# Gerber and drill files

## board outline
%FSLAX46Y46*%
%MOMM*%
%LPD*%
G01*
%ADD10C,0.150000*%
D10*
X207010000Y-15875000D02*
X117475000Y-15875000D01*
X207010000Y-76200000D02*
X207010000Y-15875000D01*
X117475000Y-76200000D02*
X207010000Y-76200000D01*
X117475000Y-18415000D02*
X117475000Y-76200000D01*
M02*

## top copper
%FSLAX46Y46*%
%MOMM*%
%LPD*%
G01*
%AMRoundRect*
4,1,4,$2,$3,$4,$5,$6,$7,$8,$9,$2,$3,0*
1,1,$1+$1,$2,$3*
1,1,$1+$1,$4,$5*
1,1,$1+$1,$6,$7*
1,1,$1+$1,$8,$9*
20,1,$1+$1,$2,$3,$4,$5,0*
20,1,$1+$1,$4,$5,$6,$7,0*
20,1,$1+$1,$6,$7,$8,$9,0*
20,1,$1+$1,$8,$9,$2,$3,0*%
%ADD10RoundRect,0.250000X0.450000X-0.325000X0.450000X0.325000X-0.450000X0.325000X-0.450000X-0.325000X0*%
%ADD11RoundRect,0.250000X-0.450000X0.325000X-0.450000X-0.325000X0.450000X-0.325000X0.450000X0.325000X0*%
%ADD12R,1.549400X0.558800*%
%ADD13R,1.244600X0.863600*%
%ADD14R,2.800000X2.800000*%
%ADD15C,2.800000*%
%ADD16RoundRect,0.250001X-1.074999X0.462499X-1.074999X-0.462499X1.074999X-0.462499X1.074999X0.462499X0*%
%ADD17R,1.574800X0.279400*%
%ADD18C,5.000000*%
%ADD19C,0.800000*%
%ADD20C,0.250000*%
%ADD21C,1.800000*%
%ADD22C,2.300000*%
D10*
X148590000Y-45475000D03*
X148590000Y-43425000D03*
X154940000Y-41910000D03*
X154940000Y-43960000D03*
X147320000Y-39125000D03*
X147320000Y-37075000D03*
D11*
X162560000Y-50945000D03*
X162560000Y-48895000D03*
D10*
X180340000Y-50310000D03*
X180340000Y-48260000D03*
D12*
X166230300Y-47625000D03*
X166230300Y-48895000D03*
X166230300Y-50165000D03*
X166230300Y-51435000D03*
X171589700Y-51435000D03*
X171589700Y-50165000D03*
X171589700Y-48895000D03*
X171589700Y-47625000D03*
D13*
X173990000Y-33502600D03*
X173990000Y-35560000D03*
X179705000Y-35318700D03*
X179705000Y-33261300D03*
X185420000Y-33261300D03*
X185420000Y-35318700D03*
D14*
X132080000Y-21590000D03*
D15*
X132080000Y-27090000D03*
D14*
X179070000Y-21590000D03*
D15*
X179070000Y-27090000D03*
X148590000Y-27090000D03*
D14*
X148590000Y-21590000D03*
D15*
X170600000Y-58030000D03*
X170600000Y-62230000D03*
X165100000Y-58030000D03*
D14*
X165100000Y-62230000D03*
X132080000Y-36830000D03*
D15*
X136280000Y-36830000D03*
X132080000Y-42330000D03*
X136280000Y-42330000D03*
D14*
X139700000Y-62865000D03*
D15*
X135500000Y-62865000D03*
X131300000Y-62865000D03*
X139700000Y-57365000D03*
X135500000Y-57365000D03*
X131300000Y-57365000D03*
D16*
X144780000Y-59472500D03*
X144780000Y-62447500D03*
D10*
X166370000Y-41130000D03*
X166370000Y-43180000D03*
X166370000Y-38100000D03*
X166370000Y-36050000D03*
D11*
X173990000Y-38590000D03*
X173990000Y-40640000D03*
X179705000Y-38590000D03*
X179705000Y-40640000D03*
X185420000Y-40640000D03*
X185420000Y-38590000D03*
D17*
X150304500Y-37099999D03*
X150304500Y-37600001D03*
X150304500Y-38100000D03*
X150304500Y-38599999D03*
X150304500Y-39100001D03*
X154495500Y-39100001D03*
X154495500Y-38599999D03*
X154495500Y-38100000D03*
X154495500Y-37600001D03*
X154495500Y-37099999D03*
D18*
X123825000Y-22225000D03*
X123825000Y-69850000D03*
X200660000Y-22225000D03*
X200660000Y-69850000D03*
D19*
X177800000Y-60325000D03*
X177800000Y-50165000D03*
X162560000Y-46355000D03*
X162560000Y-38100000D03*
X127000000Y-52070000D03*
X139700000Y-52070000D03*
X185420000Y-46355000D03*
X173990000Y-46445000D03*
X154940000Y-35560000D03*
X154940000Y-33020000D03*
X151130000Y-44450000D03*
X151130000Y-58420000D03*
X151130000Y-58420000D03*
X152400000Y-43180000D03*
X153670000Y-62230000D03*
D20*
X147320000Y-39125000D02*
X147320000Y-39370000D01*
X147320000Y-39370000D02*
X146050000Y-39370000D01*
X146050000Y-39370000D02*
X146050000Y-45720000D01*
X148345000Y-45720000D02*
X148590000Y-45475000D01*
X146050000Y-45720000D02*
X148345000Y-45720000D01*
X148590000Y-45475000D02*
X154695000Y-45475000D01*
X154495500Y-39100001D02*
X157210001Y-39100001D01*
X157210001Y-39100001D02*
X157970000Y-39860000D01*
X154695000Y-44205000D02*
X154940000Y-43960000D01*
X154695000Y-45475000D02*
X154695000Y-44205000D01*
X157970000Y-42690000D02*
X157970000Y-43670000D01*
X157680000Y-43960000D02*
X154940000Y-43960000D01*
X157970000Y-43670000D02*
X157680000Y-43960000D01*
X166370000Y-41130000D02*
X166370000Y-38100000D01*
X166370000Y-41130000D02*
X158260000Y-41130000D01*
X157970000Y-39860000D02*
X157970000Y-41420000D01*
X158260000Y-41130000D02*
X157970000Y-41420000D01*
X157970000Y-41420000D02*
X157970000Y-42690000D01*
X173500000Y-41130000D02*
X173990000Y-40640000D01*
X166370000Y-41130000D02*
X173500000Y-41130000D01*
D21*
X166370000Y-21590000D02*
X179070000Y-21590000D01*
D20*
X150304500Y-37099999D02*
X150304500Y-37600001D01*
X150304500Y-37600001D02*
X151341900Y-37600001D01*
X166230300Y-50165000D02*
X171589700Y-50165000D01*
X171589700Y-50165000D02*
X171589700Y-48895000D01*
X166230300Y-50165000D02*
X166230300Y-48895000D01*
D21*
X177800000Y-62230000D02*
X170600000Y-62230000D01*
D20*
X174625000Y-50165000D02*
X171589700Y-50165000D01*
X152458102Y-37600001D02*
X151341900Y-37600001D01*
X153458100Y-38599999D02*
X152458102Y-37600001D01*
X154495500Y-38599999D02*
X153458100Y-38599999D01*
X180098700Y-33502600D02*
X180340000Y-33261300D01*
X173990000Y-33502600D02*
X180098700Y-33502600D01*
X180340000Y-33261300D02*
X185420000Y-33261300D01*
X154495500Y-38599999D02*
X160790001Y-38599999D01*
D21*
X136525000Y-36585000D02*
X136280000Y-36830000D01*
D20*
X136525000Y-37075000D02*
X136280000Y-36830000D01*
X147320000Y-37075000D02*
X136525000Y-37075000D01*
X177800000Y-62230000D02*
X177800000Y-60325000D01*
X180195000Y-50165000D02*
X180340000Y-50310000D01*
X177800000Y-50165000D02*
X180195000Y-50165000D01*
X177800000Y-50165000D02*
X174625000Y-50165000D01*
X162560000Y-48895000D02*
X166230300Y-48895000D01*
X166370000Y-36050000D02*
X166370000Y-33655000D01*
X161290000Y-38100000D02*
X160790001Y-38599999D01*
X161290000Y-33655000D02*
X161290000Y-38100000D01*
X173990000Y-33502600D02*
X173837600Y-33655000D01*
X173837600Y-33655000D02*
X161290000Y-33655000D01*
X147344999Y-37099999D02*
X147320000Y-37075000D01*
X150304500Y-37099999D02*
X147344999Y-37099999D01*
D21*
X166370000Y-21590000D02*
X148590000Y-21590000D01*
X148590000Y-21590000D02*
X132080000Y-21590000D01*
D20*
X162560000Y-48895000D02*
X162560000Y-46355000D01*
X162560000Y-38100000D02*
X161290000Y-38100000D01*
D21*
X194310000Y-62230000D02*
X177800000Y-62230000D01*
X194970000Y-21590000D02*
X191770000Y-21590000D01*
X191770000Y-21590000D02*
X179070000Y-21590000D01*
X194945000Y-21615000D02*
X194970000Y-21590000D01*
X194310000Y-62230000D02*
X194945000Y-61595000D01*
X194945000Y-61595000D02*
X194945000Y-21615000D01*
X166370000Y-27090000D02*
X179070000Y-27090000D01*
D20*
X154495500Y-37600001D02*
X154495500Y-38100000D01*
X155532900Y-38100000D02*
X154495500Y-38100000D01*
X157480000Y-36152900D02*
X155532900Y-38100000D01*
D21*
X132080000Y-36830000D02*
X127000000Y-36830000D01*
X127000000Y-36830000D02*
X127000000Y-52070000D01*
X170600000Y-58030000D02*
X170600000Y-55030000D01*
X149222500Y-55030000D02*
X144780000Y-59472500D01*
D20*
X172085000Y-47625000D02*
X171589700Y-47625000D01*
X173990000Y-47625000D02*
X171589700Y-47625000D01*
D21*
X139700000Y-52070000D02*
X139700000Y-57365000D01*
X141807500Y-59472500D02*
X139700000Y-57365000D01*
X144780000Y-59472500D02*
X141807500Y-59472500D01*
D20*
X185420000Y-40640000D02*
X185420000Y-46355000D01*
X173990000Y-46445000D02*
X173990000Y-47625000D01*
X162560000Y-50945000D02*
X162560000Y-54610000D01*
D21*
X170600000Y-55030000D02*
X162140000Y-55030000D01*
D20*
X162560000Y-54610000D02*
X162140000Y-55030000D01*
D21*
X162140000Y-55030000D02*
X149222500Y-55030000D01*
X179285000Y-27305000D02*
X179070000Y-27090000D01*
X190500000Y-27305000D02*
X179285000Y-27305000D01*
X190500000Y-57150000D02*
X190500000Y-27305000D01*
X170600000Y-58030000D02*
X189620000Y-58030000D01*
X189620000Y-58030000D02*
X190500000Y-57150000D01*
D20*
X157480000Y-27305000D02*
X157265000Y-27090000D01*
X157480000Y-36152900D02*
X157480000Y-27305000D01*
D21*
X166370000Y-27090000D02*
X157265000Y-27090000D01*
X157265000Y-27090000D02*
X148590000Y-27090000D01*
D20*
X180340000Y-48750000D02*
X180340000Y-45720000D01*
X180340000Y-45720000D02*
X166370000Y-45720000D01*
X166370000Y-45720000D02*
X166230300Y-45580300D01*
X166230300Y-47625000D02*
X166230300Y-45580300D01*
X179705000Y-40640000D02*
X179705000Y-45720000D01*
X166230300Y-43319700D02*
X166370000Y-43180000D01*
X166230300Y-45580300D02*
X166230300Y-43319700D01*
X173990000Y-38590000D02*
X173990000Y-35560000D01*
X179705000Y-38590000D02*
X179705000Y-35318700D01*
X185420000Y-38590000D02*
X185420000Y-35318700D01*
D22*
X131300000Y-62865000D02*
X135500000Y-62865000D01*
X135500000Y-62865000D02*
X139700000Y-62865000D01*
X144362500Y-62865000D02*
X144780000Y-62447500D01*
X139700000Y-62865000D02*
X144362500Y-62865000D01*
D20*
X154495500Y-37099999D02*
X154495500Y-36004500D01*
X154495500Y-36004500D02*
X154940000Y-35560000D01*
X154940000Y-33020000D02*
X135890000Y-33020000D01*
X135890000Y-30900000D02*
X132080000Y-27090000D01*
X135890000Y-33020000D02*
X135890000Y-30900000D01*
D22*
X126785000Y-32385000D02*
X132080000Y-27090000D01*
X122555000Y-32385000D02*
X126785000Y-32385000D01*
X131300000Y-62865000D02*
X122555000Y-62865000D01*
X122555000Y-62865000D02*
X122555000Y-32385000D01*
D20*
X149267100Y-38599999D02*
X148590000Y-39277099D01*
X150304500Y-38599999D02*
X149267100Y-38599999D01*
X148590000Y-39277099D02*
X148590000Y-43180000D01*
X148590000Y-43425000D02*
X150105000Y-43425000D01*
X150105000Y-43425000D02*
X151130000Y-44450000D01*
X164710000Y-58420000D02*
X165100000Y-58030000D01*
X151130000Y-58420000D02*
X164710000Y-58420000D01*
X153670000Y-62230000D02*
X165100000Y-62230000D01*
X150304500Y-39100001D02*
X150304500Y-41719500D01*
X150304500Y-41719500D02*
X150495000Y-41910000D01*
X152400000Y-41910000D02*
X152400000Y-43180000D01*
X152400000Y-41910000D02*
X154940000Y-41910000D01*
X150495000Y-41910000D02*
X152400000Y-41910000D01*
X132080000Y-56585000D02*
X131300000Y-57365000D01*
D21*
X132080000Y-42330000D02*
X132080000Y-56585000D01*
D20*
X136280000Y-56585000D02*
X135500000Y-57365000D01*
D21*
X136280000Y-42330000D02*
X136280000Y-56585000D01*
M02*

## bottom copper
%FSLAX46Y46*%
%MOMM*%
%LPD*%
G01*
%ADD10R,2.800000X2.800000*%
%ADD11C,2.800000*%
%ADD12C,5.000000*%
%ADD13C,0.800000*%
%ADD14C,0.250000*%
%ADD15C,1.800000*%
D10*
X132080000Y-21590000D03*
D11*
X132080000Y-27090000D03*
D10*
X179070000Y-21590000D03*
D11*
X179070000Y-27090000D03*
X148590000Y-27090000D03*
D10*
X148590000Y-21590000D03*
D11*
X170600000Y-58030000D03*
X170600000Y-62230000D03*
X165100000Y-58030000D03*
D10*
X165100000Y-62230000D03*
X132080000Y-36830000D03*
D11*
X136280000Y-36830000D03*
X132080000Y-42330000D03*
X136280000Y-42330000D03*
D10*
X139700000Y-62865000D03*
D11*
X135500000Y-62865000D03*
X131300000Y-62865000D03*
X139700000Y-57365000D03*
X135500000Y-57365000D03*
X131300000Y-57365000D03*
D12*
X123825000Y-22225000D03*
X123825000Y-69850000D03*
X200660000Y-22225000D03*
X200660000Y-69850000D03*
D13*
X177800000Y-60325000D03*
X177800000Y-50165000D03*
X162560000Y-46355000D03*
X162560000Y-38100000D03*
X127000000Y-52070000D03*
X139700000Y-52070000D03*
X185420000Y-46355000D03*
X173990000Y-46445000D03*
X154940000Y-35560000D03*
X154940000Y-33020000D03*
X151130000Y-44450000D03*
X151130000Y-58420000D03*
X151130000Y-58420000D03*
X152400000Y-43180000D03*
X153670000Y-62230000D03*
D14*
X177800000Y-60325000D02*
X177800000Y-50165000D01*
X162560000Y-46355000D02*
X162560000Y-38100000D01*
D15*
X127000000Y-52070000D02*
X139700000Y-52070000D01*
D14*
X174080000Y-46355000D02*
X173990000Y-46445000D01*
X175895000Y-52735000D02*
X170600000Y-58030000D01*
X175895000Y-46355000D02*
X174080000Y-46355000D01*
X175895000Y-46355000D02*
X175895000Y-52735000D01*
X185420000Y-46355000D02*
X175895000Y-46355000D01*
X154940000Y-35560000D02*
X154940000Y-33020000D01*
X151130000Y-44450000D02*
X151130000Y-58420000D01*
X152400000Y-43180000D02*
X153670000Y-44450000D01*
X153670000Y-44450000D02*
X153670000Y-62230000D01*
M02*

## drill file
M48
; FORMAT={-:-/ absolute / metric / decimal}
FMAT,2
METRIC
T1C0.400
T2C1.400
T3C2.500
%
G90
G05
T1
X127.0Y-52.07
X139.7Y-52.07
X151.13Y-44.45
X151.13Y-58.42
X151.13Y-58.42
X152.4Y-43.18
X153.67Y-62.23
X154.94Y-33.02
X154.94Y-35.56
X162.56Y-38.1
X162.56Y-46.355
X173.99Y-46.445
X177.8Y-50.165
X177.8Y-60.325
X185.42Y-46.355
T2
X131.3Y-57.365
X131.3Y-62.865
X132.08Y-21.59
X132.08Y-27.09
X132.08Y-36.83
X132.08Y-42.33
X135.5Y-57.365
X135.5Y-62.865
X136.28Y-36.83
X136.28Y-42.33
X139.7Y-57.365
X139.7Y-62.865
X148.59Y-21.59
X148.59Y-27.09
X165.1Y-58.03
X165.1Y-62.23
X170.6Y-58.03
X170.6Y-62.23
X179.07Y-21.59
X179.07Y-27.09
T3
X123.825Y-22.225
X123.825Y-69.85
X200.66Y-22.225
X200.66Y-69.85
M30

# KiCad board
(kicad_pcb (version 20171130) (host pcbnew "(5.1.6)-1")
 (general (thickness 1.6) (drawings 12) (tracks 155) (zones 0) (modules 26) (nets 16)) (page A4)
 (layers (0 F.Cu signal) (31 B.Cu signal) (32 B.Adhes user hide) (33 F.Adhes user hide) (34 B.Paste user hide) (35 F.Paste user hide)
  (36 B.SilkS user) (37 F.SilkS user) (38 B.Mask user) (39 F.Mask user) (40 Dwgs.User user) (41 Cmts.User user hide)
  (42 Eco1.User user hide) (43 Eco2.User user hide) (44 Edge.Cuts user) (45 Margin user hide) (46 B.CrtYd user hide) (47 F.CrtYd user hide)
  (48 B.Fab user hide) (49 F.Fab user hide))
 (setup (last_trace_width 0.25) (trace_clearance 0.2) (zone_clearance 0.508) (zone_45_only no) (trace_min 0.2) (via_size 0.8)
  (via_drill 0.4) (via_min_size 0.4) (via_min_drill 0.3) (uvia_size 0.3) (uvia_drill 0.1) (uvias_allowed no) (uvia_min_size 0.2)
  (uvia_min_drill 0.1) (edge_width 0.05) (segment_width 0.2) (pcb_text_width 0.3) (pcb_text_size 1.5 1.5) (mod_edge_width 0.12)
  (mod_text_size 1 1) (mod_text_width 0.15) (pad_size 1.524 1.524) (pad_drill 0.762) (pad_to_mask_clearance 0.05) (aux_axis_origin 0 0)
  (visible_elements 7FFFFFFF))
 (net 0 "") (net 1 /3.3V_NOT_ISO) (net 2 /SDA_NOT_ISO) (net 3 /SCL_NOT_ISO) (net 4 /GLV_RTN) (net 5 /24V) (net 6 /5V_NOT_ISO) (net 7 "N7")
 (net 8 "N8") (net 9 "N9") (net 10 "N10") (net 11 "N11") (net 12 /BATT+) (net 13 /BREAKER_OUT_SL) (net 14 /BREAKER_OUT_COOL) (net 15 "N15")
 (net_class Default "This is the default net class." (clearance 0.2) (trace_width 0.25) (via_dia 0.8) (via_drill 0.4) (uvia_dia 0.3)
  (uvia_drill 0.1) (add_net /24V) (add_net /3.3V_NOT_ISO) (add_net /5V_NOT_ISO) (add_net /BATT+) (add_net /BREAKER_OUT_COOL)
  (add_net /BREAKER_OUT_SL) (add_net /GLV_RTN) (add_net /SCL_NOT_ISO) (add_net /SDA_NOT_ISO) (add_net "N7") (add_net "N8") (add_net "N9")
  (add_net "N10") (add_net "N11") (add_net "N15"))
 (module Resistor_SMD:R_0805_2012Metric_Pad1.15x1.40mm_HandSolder (layer F.Cu) (at 148.59 44.45 90)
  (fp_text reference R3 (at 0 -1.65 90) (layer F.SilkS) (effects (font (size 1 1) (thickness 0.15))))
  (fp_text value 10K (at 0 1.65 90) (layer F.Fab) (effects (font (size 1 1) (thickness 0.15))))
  (pad 1 smd roundrect (at -1.025 0 90) (size 1.15 1.4) (layers F.Cu F.Paste F.Mask) (roundrect_rratio 0.217391) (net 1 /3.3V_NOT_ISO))
  (pad 2 smd roundrect (at 1.025 0 90) (size 1.15 1.4) (layers F.Cu F.Paste F.Mask) (roundrect_rratio 0.217391) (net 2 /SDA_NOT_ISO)))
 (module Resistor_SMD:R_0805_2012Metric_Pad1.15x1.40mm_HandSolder (layer F.Cu) (at 154.94 42.935 90)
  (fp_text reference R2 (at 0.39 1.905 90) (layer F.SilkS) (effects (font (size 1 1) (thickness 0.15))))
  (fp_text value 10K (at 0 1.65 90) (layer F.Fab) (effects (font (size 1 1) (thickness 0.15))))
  (pad 2 smd roundrect (at 1.025 0 90) (size 1.15 1.4) (layers F.Cu F.Paste F.Mask) (roundrect_rratio 0.217391) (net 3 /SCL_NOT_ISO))
  (pad 1 smd roundrect (at -1.025 0 90) (size 1.15 1.4) (layers F.Cu F.Paste F.Mask) (roundrect_rratio 0.217391) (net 1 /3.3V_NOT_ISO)))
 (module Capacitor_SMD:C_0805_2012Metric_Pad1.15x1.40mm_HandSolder (layer F.Cu) (at 147.32 38.1 90)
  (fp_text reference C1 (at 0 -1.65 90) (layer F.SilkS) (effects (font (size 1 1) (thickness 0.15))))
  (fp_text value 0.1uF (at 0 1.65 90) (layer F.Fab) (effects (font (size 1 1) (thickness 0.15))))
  (pad 1 smd roundrect (at -1.025 0 90) (size 1.15 1.4) (layers F.Cu F.Paste F.Mask) (roundrect_rratio 0.217391) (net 1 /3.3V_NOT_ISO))
  (pad 2 smd roundrect (at 1.025 0 90) (size 1.15 1.4) (layers F.Cu F.Paste F.Mask) (roundrect_rratio 0.217391) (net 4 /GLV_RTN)))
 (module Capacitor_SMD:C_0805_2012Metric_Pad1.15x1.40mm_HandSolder (layer F.Cu) (at 162.56 49.92 270)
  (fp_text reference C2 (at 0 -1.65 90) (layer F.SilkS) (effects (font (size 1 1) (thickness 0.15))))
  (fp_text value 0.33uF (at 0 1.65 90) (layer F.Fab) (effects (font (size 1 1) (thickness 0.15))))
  (pad 2 smd roundrect (at 1.025 0 270) (size 1.15 1.4) (layers F.Cu F.Paste F.Mask) (roundrect_rratio 0.217391) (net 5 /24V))
  (pad 1 smd roundrect (at -1.025 0 270) (size 1.15 1.4) (layers F.Cu F.Paste F.Mask) (roundrect_rratio 0.217391) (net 4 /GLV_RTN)))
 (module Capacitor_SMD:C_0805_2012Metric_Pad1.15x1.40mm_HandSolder (layer F.Cu) (at 180.34 49.285 90)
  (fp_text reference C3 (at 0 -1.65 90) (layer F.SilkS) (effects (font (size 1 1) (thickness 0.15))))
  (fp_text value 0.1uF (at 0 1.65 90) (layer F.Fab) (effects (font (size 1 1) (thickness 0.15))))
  (pad 1 smd roundrect (at -1.025 0 90) (size 1.15 1.4) (layers F.Cu F.Paste F.Mask) (roundrect_rratio 0.217391) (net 4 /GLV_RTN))
  (pad 2 smd roundrect (at 1.025 0 90) (size 1.15 1.4) (layers F.Cu F.Paste F.Mask) (roundrect_rratio 0.217391) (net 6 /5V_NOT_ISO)))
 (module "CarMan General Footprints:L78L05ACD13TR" (layer F.Cu) (at 168.91 49.53)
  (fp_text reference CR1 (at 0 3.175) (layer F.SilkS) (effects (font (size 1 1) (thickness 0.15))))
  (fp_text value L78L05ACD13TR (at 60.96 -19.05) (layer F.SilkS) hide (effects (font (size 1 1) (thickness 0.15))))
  (pad 1 smd rect (at -2.6797 -1.905) (size 1.5494 0.5588) (layers F.Cu F.Paste F.Mask) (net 6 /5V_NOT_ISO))
  (pad 2 smd rect (at -2.6797 -0.635) (size 1.5494 0.5588) (layers F.Cu F.Paste F.Mask) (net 4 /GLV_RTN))
  (pad 3 smd rect (at -2.6797 0.635) (size 1.5494 0.5588) (layers F.Cu F.Paste F.Mask) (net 4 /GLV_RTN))
  (pad 4 smd rect (at -2.6797 1.905) (size 1.5494 0.5588) (layers F.Cu F.Paste F.Mask) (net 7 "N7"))
  (pad 5 smd rect (at 2.6797 1.905) (size 1.5494 0.5588) (layers F.Cu F.Paste F.Mask) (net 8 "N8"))
  (pad 6 smd rect (at 2.6797 0.635) (size 1.5494 0.5588) (layers F.Cu F.Paste F.Mask) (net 4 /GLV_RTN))
  (pad 7 smd rect (at 2.6797 -0.635) (size 1.5494 0.5588) (layers F.Cu F.Paste F.Mask) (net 4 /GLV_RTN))
  (pad 8 smd rect (at 2.6797 -1.905) (size 1.5494 0.5588) (layers F.Cu F.Paste F.Mask) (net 5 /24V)))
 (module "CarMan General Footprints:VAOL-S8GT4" (layer F.Cu) (at 173.99 34.5313 270)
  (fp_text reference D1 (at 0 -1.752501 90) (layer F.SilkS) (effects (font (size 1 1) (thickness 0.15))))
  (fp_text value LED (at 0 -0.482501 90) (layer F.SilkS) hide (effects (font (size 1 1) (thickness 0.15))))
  (pad 1 smd rect (at -1.0287 0 270) (size 0.8636 1.2446) (layers F.Cu F.Paste F.Mask) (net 4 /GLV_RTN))
  (pad 2 smd rect (at 1.0287 0 270) (size 0.8636 1.2446) (layers F.Cu F.Paste F.Mask) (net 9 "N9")))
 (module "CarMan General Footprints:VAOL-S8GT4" (layer F.Cu) (at 179.705 34.29 270)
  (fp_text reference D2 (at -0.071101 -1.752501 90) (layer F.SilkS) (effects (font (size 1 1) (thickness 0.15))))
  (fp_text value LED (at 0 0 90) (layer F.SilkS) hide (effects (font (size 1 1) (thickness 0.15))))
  (pad 2 smd rect (at 1.0287 0 270) (size 0.8636 1.2446) (layers F.Cu F.Paste F.Mask) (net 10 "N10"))
  (pad 1 smd rect (at -1.0287 0 270) (size 0.8636 1.2446) (layers F.Cu F.Paste F.Mask) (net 4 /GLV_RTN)))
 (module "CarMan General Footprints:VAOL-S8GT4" (layer F.Cu) (at 185.42 34.29 270)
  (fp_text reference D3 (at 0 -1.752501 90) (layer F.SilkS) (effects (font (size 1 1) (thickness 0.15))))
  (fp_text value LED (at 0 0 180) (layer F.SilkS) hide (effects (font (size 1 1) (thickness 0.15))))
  (pad 1 smd rect (at -1.0287 0 270) (size 0.8636 1.2446) (layers F.Cu F.Paste F.Mask) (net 4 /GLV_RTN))
  (pad 2 smd rect (at 1.0287 0 270) (size 0.8636 1.2446) (layers F.Cu F.Paste F.Mask) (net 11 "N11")))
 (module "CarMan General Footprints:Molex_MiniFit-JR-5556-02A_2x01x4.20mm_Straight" (layer F.Cu) (at 132.08 21.59)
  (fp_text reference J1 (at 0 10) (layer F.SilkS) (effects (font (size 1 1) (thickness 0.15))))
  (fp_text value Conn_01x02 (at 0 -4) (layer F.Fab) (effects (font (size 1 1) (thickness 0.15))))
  (pad 1 thru_hole rect (at 0 0) (size 2.8 2.8) (drill 1.4) (layers *.Cu *.Mask) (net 4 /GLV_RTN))
  (pad 2 thru_hole circle (at 0 5.5) (size 2.8 2.8) (drill 1.4) (layers *.Cu *.Mask) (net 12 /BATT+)))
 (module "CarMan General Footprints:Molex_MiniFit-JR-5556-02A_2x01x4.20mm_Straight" (layer F.Cu) (at 179.07 21.59)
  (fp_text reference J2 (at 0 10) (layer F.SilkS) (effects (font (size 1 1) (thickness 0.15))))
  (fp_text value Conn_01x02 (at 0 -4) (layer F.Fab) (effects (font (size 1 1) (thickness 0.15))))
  (pad 1 thru_hole rect (at 0 0) (size 2.8 2.8) (drill 1.4) (layers *.Cu *.Mask) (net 4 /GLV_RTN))
  (pad 2 thru_hole circle (at 0 5.5) (size 2.8 2.8) (drill 1.4) (layers *.Cu *.Mask) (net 5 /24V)))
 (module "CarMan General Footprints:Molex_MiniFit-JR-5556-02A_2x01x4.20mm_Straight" (layer F.Cu) (at 148.59 21.59)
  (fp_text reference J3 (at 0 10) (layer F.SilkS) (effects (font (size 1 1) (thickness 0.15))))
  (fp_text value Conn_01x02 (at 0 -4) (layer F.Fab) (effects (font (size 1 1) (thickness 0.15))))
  (pad 2 thru_hole circle (at 0 5.5) (size 2.8 2.8) (drill 1.4) (layers *.Cu *.Mask) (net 5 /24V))
  (pad 1 thru_hole rect (at 0 0) (size 2.8 2.8) (drill 1.4) (layers *.Cu *.Mask) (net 4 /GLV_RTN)))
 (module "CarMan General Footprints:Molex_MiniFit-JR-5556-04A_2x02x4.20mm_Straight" (layer F.Cu) (at 165.1 62.23 90)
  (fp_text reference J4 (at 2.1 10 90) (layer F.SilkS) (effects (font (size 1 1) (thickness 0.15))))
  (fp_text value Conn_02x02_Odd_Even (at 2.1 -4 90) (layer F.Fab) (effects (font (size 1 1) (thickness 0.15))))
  (pad 4 thru_hole circle (at 4.2 5.5 90) (size 2.8 2.8) (drill 1.4) (layers *.Cu *.Mask) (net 5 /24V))
  (pad 3 thru_hole circle (at 0 5.5 90) (size 2.8 2.8) (drill 1.4) (layers *.Cu *.Mask) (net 4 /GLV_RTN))
  (pad 2 thru_hole circle (at 4.2 0 90) (size 2.8 2.8) (drill 1.4) (layers *.Cu *.Mask) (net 2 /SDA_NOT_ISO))
  (pad 1 thru_hole rect (at 0 0 90) (size 2.8 2.8) (drill 1.4) (layers *.Cu *.Mask) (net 3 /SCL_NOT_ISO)))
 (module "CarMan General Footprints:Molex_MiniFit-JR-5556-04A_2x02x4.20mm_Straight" (layer F.Cu) (at 132.08 36.83)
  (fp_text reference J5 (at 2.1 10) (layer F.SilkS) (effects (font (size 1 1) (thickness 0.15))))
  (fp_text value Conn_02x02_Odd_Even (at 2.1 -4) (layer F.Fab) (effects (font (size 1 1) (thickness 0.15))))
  (pad 1 thru_hole rect (at 0 0) (size 2.8 2.8) (drill 1.4) (layers *.Cu *.Mask) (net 5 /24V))
  (pad 2 thru_hole circle (at 4.2 0) (size 2.8 2.8) (drill 1.4) (layers *.Cu *.Mask) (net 4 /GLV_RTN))
  (pad 3 thru_hole circle (at 0 5.5) (size 2.8 2.8) (drill 1.4) (layers *.Cu *.Mask) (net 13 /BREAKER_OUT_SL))
  (pad 4 thru_hole circle (at 4.2 5.5) (size 2.8 2.8) (drill 1.4) (layers *.Cu *.Mask) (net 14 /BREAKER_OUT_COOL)))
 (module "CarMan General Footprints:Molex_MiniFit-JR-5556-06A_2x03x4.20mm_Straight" (layer F.Cu) (at 139.7 62.865 180)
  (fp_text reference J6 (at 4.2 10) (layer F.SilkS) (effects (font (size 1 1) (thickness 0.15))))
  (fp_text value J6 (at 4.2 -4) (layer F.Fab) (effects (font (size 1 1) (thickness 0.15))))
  (pad 1 thru_hole rect (at 0 0 180) (size 2.8 2.8) (drill 1.4) (layers *.Cu *.Mask) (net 12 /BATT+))
  (pad 2 thru_hole circle (at 4.2 0 180) (size 2.8 2.8) (drill 1.4) (layers *.Cu *.Mask) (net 12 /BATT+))
  (pad 3 thru_hole circle (at 8.4 0 180) (size 2.8 2.8) (drill 1.4) (layers *.Cu *.Mask) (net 12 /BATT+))
  (pad 4 thru_hole circle (at 0 5.5 180) (size 2.8 2.8) (drill 1.4) (layers *.Cu *.Mask) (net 5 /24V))
  (pad 5 thru_hole circle (at 4.2 5.5 180) (size 2.8 2.8) (drill 1.4) (layers *.Cu *.Mask) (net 14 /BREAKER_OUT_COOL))
  (pad 6 thru_hole circle (at 8.4 5.5 180) (size 2.8 2.8) (drill 1.4) (layers *.Cu *.Mask) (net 13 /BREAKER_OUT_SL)))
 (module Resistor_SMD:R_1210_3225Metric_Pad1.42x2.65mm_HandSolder (layer F.Cu) (at 144.78 60.96 270)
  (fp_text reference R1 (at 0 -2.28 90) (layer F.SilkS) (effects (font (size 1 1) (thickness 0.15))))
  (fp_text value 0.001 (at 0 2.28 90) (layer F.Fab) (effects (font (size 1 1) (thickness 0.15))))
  (pad 1 smd roundrect (at -1.4875 0 270) (size 1.425 2.65) (layers F.Cu F.Paste F.Mask) (roundrect_rratio 0.175439) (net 5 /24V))
  (pad 2 smd roundrect (at 1.4875 0 270) (size 1.425 2.65) (layers F.Cu F.Paste F.Mask) (roundrect_rratio 0.175439) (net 12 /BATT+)))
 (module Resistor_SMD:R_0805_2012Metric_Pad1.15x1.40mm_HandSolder (layer F.Cu) (at 166.37 42.155 90)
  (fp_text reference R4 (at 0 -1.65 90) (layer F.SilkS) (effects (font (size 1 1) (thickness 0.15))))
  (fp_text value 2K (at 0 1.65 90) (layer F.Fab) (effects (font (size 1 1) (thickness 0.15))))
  (pad 2 smd roundrect (at 1.025 0 90) (size 1.15 1.4) (layers F.Cu F.Paste F.Mask) (roundrect_rratio 0.217391) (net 1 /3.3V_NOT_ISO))
  (pad 1 smd roundrect (at -1.025 0 90) (size 1.15 1.4) (layers F.Cu F.Paste F.Mask) (roundrect_rratio 0.217391) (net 6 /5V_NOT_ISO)))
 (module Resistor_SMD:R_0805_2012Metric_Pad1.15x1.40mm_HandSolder (layer F.Cu) (at 166.37 37.075 90)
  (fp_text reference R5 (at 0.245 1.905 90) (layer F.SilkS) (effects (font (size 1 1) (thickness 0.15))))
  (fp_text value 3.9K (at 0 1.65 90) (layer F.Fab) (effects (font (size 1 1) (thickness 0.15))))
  (pad 1 smd roundrect (at -1.025 0 90) (size 1.15 1.4) (layers F.Cu F.Paste F.Mask) (roundrect_rratio 0.217391) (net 1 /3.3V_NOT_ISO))
  (pad 2 smd roundrect (at 1.025 0 90) (size 1.15 1.4) (layers F.Cu F.Paste F.Mask) (roundrect_rratio 0.217391) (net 4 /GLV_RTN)))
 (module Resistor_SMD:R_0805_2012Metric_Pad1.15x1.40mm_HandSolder (layer F.Cu) (at 173.99 39.615 270)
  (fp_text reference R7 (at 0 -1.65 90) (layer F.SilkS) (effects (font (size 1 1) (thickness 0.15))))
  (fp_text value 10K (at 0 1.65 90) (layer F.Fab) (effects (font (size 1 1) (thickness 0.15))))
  (pad 1 smd roundrect (at -1.025 0 270) (size 1.15 1.4) (layers F.Cu F.Paste F.Mask) (roundrect_rratio 0.217391) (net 9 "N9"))
  (pad 2 smd roundrect (at 1.025 0 270) (size 1.15 1.4) (layers F.Cu F.Paste F.Mask) (roundrect_rratio 0.217391) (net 1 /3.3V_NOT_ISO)))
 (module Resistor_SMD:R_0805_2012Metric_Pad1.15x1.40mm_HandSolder (layer F.Cu) (at 179.705 39.615 270)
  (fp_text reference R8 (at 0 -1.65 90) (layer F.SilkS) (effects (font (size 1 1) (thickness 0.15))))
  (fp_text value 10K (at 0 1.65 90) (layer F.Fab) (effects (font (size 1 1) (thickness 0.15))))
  (pad 1 smd roundrect (at -1.025 0 270) (size 1.15 1.4) (layers F.Cu F.Paste F.Mask) (roundrect_rratio 0.217391) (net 10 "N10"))
  (pad 2 smd roundrect (at 1.025 0 270) (size 1.15 1.4) (layers F.Cu F.Paste F.Mask) (roundrect_rratio 0.217391) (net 6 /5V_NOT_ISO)))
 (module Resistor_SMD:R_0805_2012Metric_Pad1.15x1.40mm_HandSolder (layer F.Cu) (at 185.42 39.615 270)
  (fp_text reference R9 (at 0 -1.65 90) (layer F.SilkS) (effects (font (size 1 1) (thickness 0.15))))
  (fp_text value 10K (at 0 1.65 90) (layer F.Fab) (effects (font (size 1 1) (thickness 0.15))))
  (pad 2 smd roundrect (at 1.025 0 270) (size 1.15 1.4) (layers F.Cu F.Paste F.Mask) (roundrect_rratio 0.217391) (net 5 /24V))
  (pad 1 smd roundrect (at -1.025 0 270) (size 1.15 1.4) (layers F.Cu F.Paste F.Mask) (roundrect_rratio 0.217391) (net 11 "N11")))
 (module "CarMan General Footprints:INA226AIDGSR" (layer F.Cu) (at 152.4 38.1)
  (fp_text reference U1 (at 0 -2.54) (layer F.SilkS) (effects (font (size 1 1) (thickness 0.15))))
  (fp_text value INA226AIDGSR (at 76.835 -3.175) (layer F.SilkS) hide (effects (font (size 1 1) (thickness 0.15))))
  (pad 1 smd rect (at -2.0955 -1.000001) (size 1.5748 0.2794) (layers F.Cu F.Paste F.Mask) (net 4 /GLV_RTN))
  (pad 2 smd rect (at -2.0955 -0.499999) (size 1.5748 0.2794) (layers F.Cu F.Paste F.Mask) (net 4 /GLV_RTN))
  (pad 3 smd rect (at -2.0955 0) (size 1.5748 0.2794) (layers F.Cu F.Paste F.Mask) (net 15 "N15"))
  (pad 4 smd rect (at -2.0955 0.499999) (size 1.5748 0.2794) (layers F.Cu F.Paste F.Mask) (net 2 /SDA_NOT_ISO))
  (pad 5 smd rect (at -2.0955 1.000001) (size 1.5748 0.2794) (layers F.Cu F.Paste F.Mask) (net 3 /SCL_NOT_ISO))
  (pad 6 smd rect (at 2.0955 1.000001) (size 1.5748 0.2794) (layers F.Cu F.Paste F.Mask) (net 1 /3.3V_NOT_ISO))
  (pad 7 smd rect (at 2.0955 0.499999) (size 1.5748 0.2794) (layers F.Cu F.Paste F.Mask) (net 4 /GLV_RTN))
  (pad 8 smd rect (at 2.0955 0) (size 1.5748 0.2794) (layers F.Cu F.Paste F.Mask) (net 5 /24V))
  (pad 9 smd rect (at 2.0955 -0.499999) (size 1.5748 0.2794) (layers F.Cu F.Paste F.Mask) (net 5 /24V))
  (pad 10 smd rect (at 2.0955 -1.000001) (size 1.5748 0.2794) (layers F.Cu F.Paste F.Mask) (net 12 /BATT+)))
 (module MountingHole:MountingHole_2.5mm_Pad (layer F.Cu) (at 123.825 22.225)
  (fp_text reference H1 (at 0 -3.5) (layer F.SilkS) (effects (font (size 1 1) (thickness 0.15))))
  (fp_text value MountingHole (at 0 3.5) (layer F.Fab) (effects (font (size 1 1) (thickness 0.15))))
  (pad 1 thru_hole circle (at 0 0) (size 5 5) (drill 2.5) (layers *.Cu *.Mask)))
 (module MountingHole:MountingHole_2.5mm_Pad (layer F.Cu) (at 123.825 69.85)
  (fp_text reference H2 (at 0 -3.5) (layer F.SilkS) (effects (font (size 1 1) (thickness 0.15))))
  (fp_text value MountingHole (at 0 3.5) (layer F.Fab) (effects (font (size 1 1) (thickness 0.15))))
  (pad 1 thru_hole circle (at 0 0) (size 5 5) (drill 2.5) (layers *.Cu *.Mask)))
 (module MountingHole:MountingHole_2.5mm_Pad (layer F.Cu) (at 200.66 22.225)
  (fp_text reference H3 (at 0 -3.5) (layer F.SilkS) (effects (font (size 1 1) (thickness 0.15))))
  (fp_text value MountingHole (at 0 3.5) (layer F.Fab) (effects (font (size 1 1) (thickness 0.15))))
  (pad 1 thru_hole circle (at 0 0) (size 5 5) (drill 2.5) (layers *.Cu *.Mask)))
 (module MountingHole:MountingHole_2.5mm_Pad (layer F.Cu) (at 200.66 69.85)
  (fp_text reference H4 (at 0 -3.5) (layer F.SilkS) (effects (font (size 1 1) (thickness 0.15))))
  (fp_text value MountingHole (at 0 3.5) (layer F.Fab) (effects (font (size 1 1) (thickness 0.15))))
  (pad 1 thru_hole circle (at 0 0) (size 5 5) (drill 2.5) (layers *.Cu *.Mask)))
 (gr_line (start 207.01 15.875) (end 117.475 15.875) (layer Edge.Cuts) (width 0.15))
 (gr_line (start 207.01 76.2) (end 207.01 15.875) (layer Edge.Cuts) (width 0.15))
 (gr_line (start 117.475 76.2) (end 207.01 76.2) (layer Edge.Cuts) (width 0.15))
 (gr_line (start 117.475 18.415) (end 117.475 76.2) (layer Edge.Cuts) (width 0.15))
 (segment (start 147.32 39.125) (end 147.32 39.37) (width 0.25) (layer F.Cu) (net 1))
 (segment (start 147.32 39.37) (end 146.05 39.37) (width 0.25) (layer F.Cu) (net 1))
 (segment (start 146.05 39.37) (end 146.05 45.72) (width 0.25) (layer F.Cu) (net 1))
 (segment (start 148.345 45.72) (end 148.59 45.475) (width 0.25) (layer F.Cu) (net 1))
 (segment (start 146.05 45.72) (end 148.345 45.72) (width 0.25) (layer F.Cu) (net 1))
 (segment (start 148.59 45.475) (end 154.695 45.475) (width 0.25) (layer F.Cu) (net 1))
 (segment (start 154.4955 39.100001) (end 157.210001 39.100001) (width 0.25) (layer F.Cu) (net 1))
 (segment (start 157.210001 39.100001) (end 157.97 39.86) (width 0.25) (layer F.Cu) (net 1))
 (segment (start 154.695 44.205) (end 154.94 43.96) (width 0.25) (layer F.Cu) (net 1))
 (segment (start 154.695 45.475) (end 154.695 44.205) (width 0.25) (layer F.Cu) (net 1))
 (segment (start 157.97 42.69) (end 157.97 43.67) (width 0.25) (layer F.Cu) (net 1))
 (segment (start 157.68 43.96) (end 154.94 43.96) (width 0.25) (layer F.Cu) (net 1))
 (segment (start 157.97 43.67) (end 157.68 43.96) (width 0.25) (layer F.Cu) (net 1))
 (segment (start 166.37 41.13) (end 166.37 38.1) (width 0.25) (layer F.Cu) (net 1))
 (segment (start 166.37 41.13) (end 158.26 41.13) (width 0.25) (layer F.Cu) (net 1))
 (segment (start 157.97 39.86) (end 157.97 41.42) (width 0.25) (layer F.Cu) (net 1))
 (segment (start 158.26 41.13) (end 157.97 41.42) (width 0.25) (layer F.Cu) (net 1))
 (segment (start 157.97 41.42) (end 157.97 42.69) (width 0.25) (layer F.Cu) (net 1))
 (segment (start 173.5 41.13) (end 173.99 40.64) (width 0.25) (layer F.Cu) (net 1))
 (segment (start 166.37 41.13) (end 173.5 41.13) (width 0.25) (layer F.Cu) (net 1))
 (segment (start 166.37 21.59) (end 179.07 21.59) (width 1.8) (layer F.Cu) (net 4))
 (segment (start 150.3045 37.099999) (end 150.3045 37.600001) (width 0.25) (layer F.Cu) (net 4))
 (segment (start 150.3045 37.600001) (end 151.3419 37.600001) (width 0.25) (layer F.Cu) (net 4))
 (segment (start 166.2303 50.165) (end 171.5897 50.165) (width 0.25) (layer F.Cu) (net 4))
 (segment (start 171.5897 50.165) (end 171.5897 48.895) (width 0.25) (layer F.Cu) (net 4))
 (segment (start 166.2303 50.165) (end 166.2303 48.895) (width 0.25) (layer F.Cu) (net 4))
 (segment (start 177.8 62.23) (end 170.6 62.23) (width 1.8) (layer F.Cu) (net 4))
 (segment (start 174.625 50.165) (end 171.5897 50.165) (width 0.25) (layer F.Cu) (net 4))
 (segment (start 152.458102 37.600001) (end 151.3419 37.600001) (width 0.25) (layer F.Cu) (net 4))
 (segment (start 153.4581 38.599999) (end 152.458102 37.600001) (width 0.25) (layer F.Cu) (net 4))
 (segment (start 154.4955 38.599999) (end 153.4581 38.599999) (width 0.25) (layer F.Cu) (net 4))
 (segment (start 180.0987 33.5026) (end 180.34 33.2613) (width 0.25) (layer F.Cu) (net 4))
 (segment (start 173.99 33.5026) (end 180.0987 33.5026) (width 0.25) (layer F.Cu) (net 4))
 (segment (start 180.34 33.2613) (end 185.42 33.2613) (width 0.25) (layer F.Cu) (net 4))
 (segment (start 154.4955 38.599999) (end 160.790001 38.599999) (width 0.25) (layer F.Cu) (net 4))
 (segment (start 136.525 36.585) (end 136.28 36.83) (width 1.8) (layer F.Cu) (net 4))
 (segment (start 136.525 37.075) (end 136.28 36.83) (width 0.25) (layer F.Cu) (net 4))
 (segment (start 147.32 37.075) (end 136.525 37.075) (width 0.25) (layer F.Cu) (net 4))
 (via (at 177.8 60.325) (size 0.8) (drill 0.4) (layers F.Cu B.Cu) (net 4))
 (segment (start 177.8 62.23) (end 177.8 60.325) (width 0.25) (layer F.Cu) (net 4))
 (via (at 177.8 50.165) (size 0.8) (drill 0.4) (layers F.Cu B.Cu) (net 4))
 (segment (start 177.8 60.325) (end 177.8 50.165) (width 0.25) (layer B.Cu) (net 4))
 (segment (start 180.195 50.165) (end 180.34 50.31) (width 0.25) (layer F.Cu) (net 4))
 (segment (start 177.8 50.165) (end 180.195 50.165) (width 0.25) (layer F.Cu) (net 4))
 (segment (start 177.8 50.165) (end 174.625 50.165) (width 0.25) (layer F.Cu) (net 4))
 (segment (start 162.56 48.895) (end 166.2303 48.895) (width 0.25) (layer F.Cu) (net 4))
 (segment (start 166.37 36.05) (end 166.37 33.655) (width 0.25) (layer F.Cu) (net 4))
 (segment (start 161.29 38.1) (end 160.790001 38.599999) (width 0.25) (layer F.Cu) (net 4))
 (segment (start 161.29 33.655) (end 161.29 38.1) (width 0.25) (layer F.Cu) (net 4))
 (segment (start 173.99 33.5026) (end 173.8376 33.655) (width 0.25) (layer F.Cu) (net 4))
 (segment (start 173.8376 33.655) (end 161.29 33.655) (width 0.25) (layer F.Cu) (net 4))
 (segment (start 147.344999 37.099999) (end 147.32 37.075) (width 0.25) (layer F.Cu) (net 4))
 (segment (start 150.3045 37.099999) (end 147.344999 37.099999) (width 0.25) (layer F.Cu) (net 4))
 (segment (start 166.37 21.59) (end 148.59 21.59) (width 1.8) (layer F.Cu) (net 4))
 (segment (start 148.59 21.59) (end 132.08 21.59) (width 1.8) (layer F.Cu) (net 4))
 (via (at 162.56 46.355) (size 0.8) (drill 0.4) (layers F.Cu B.Cu) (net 4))
 (segment (start 162.56 48.895) (end 162.56 46.355) (width 0.25) (layer F.Cu) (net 4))
 (via (at 162.56 38.1) (size 0.8) (drill 0.4) (layers F.Cu B.Cu) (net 4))
 (segment (start 162.56 46.355) (end 162.56 38.1) (width 0.25) (layer B.Cu) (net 4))
 (segment (start 162.56 38.1) (end 161.29 38.1) (width 0.25) (layer F.Cu) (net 4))
 (segment (start 194.31 62.23) (end 177.8 62.23) (width 1.8) (layer F.Cu) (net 4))
 (segment (start 194.97 21.59) (end 191.77 21.59) (width 1.8) (layer F.Cu) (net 4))
 (segment (start 191.77 21.59) (end 179.07 21.59) (width 1.8) (layer F.Cu) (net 4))
 (segment (start 194.945 21.615) (end 194.97 21.59) (width 1.8) (layer F.Cu) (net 4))
 (segment (start 194.31 62.23) (end 194.945 61.595) (width 1.8) (layer F.Cu) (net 4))
 (segment (start 194.945 61.595) (end 194.945 21.615) (width 1.8) (layer F.Cu) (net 4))
 (segment (start 166.37 27.09) (end 179.07 27.09) (width 1.8) (layer F.Cu) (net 5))
 (segment (start 154.4955 37.600001) (end 154.4955 38.1) (width 0.25) (layer F.Cu) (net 5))
 (segment (start 155.5329 38.1) (end 154.4955 38.1) (width 0.25) (layer F.Cu) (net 5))
 (segment (start 157.48 36.1529) (end 155.5329 38.1) (width 0.25) (layer F.Cu) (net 5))
 (segment (start 132.08 36.83) (end 127 36.83) (width 1.8) (layer F.Cu) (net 5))
 (via (at 127 52.07) (size 0.8) (drill 0.4) (layers F.Cu B.Cu) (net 5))
 (segment (start 127 36.83) (end 127 52.07) (width 1.8) (layer F.Cu) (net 5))
 (via (at 139.7 52.07) (size 0.8) (drill 0.4) (layers F.Cu B.Cu) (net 5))
 (segment (start 127 52.07) (end 139.7 52.07) (width 1.8) (layer B.Cu) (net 5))
 (segment (start 170.6 58.03) (end 170.6 55.03) (width 1.8) (layer F.Cu) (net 5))
 (segment (start 149.2225 55.03) (end 144.78 59.4725) (width 1.8) (layer F.Cu) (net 5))
 (segment (start 172.085 47.625) (end 171.5897 47.625) (width 0.25) (layer F.Cu) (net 5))
 (segment (start 173.99 47.625) (end 171.5897 47.625) (width 0.25) (layer F.Cu) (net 5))
 (segment (start 139.7 52.07) (end 139.7 57.365) (width 1.8) (layer F.Cu) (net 5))
 (segment (start 141.8075 59.4725) (end 139.7 57.365) (width 1.8) (layer F.Cu) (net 5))
 (segment (start 144.78 59.4725) (end 141.8075 59.4725) (width 1.8) (layer F.Cu) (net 5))
 (via (at 185.42 46.355) (size 0.8) (drill 0.4) (layers F.Cu B.Cu) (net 5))
 (segment (start 185.42 40.64) (end 185.42 46.355) (width 0.25) (layer F.Cu) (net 5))
 (via (at 173.99 46.445) (size 0.8) (drill 0.4) (layers F.Cu B.Cu) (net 5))
 (segment (start 174.08 46.355) (end 173.99 46.445) (width 0.25) (layer B.Cu) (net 5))
 (segment (start 173.99 46.445) (end 173.99 47.625) (width 0.25) (layer F.Cu) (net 5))
 (segment (start 162.56 50.945) (end 162.56 54.61) (width 0.25) (layer F.Cu) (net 5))
 (segment (start 170.6 55.03) (end 162.14 55.03) (width 1.8) (layer F.Cu) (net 5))
 (segment (start 162.56 54.61) (end 162.14 55.03) (width 0.25) (layer F.Cu) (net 5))
 (segment (start 162.14 55.03) (end 149.2225 55.03) (width 1.8) (layer F.Cu) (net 5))
 (segment (start 179.285 27.305) (end 179.07 27.09) (width 1.8) (layer F.Cu) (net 5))
 (segment (start 190.5 27.305) (end 179.285 27.305) (width 1.8) (layer F.Cu) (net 5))
 (segment (start 190.5 57.15) (end 190.5 27.305) (width 1.8) (layer F.Cu) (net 5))
 (segment (start 170.6 58.03) (end 189.62 58.03) (width 1.8) (layer F.Cu) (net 5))
 (segment (start 189.62 58.03) (end 190.5 57.15) (width 1.8) (layer F.Cu) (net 5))
 (segment (start 175.895 52.735) (end 170.6 58.03) (width 0.25) (layer B.Cu) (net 5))
 (segment (start 175.895 46.355) (end 174.08 46.355) (width 0.25) (layer B.Cu) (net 5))
 (segment (start 175.895 46.355) (end 175.895 52.735) (width 0.25) (layer B.Cu) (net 5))
 (segment (start 185.42 46.355) (end 175.895 46.355) (width 0.25) (layer B.Cu) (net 5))
 (segment (start 157.48 27.305) (end 157.265 27.09) (width 0.25) (layer F.Cu) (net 5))
 (segment (start 157.48 36.1529) (end 157.48 27.305) (width 0.25) (layer F.Cu) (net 5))
 (segment (start 166.37 27.09) (end 157.265 27.09) (width 1.8) (layer F.Cu) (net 5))
 (segment (start 157.265 27.09) (end 148.59 27.09) (width 1.8) (layer F.Cu) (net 5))
 (segment (start 180.34 48.75) (end 180.34 45.72) (width 0.25) (layer F.Cu) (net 6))
 (segment (start 180.34 45.72) (end 166.37 45.72) (width 0.25) (layer F.Cu) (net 6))
 (segment (start 166.37 45.72) (end 166.2303 45.5803) (width 0.25) (layer F.Cu) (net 6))
 (segment (start 166.2303 47.625) (end 166.2303 45.5803) (width 0.25) (layer F.Cu) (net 6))
 (segment (start 179.705 40.64) (end 179.705 45.72) (width 0.25) (layer F.Cu) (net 6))
 (segment (start 166.2303 43.3197) (end 166.37 43.18) (width 0.25) (layer F.Cu) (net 6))
 (segment (start 166.2303 45.5803) (end 166.2303 43.3197) (width 0.25) (layer F.Cu) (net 6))
 (segment (start 173.99 38.59) (end 173.99 35.56) (width 0.25) (layer F.Cu) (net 9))
 (segment (start 179.705 38.59) (end 179.705 35.3187) (width 0.25) (layer F.Cu) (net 10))
 (segment (start 185.42 38.59) (end 185.42 35.3187) (width 0.25) (layer F.Cu) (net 11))
 (segment (start 131.3 62.865) (end 135.5 62.865) (width 2.3) (layer F.Cu) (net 12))
 (segment (start 135.5 62.865) (end 139.7 62.865) (width 2.3) (layer F.Cu) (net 12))
 (segment (start 144.3625 62.865) (end 144.78 62.4475) (width 2.3) (layer F.Cu) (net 12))
 (segment (start 139.7 62.865) (end 144.3625 62.865) (width 2.3) (layer F.Cu) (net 12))
 (via (at 154.94 35.56) (size 0.8) (drill 0.4) (layers F.Cu B.Cu) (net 12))
 (segment (start 154.4955 37.099999) (end 154.4955 36.0045) (width 0.25) (layer F.Cu) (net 12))
 (segment (start 154.4955 36.0045) (end 154.94 35.56) (width 0.25) (layer F.Cu) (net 12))
 (via (at 154.94 33.02) (size 0.8) (drill 0.4) (layers F.Cu B.Cu) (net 12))
 (segment (start 154.94 35.56) (end 154.94 33.02) (width 0.25) (layer B.Cu) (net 12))
 (segment (start 154.94 33.02) (end 135.89 33.02) (width 0.25) (layer F.Cu) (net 12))
 (segment (start 135.89 30.9) (end 132.08 27.09) (width 0.25) (layer F.Cu) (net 12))
 (segment (start 135.89 33.02) (end 135.89 30.9) (width 0.25) (layer F.Cu) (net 12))
 (segment (start 126.785 32.385) (end 132.08 27.09) (width 2.3) (layer F.Cu) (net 12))
 (segment (start 122.555 32.385) (end 126.785 32.385) (width 2.3) (layer F.Cu) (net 12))
 (segment (start 131.3 62.865) (end 122.555 62.865) (width 2.3) (layer F.Cu) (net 12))
 (segment (start 122.555 62.865) (end 122.555 32.385) (width 2.3) (layer F.Cu) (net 12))
 (segment (start 149.2671 38.599999) (end 148.59 39.277099) (width 0.25) (layer F.Cu) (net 2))
 (segment (start 150.3045 38.599999) (end 149.2671 38.599999) (width 0.25) (layer F.Cu) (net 2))
 (segment (start 148.59 39.277099) (end 148.59 43.18) (width 0.25) (layer F.Cu) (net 2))
 (via (at 151.13 44.45) (size 0.8) (drill 0.4) (layers F.Cu B.Cu) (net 2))
 (segment (start 148.59 43.425) (end 150.105 43.425) (width 0.25) (layer F.Cu) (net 2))
 (segment (start 150.105 43.425) (end 151.13 44.45) (width 0.25) (layer F.Cu) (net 2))
 (segment (start 151.13 44.45) (end 151.13 58.42) (width 0.25) (layer B.Cu) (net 2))
 (via (at 151.13 58.42) (size 0.8) (drill 0.4) (layers F.Cu B.Cu) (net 2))
 (via (at 151.13 58.42) (size 0.8) (drill 0.4) (layers F.Cu B.Cu) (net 2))
 (segment (start 164.71 58.42) (end 165.1 58.03) (width 0.25) (layer F.Cu) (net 2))
 (segment (start 151.13 58.42) (end 164.71 58.42) (width 0.25) (layer F.Cu) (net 2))
 (via (at 152.4 43.18) (size 0.8) (drill 0.4) (layers F.Cu B.Cu) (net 3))
 (via (at 153.67 62.23) (size 0.8) (drill 0.4) (layers F.Cu B.Cu) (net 3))
 (segment (start 152.4 43.18) (end 153.67 44.45) (width 0.25) (layer B.Cu) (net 3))
 (segment (start 153.67 44.45) (end 153.67 62.23) (width 0.25) (layer B.Cu) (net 3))
 (segment (start 153.67 62.23) (end 165.1 62.23) (width 0.25) (layer F.Cu) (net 3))
 (segment (start 150.3045 39.100001) (end 150.3045 41.7195) (width 0.25) (layer F.Cu) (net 3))
 (segment (start 150.3045 41.7195) (end 150.495 41.91) (width 0.25) (layer F.Cu) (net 3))
 (segment (start 152.4 41.91) (end 152.4 43.18) (width 0.25) (layer F.Cu) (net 3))
 (segment (start 152.4 41.91) (end 154.94 41.91) (width 0.25) (layer F.Cu) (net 3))
 (segment (start 150.495 41.91) (end 152.4 41.91) (width 0.25) (layer F.Cu) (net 3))
 (segment (start 132.08 56.585) (end 131.3 57.365) (width 0.25) (layer F.Cu) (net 13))
 (segment (start 132.08 42.33) (end 132.08 56.585) (width 1.8) (layer F.Cu) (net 13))
 (segment (start 136.28 56.585) (end 135.5 57.365) (width 0.25) (layer F.Cu) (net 14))
 (segment (start 136.28 42.33) (end 136.28 56.585) (width 1.8) (layer F.Cu) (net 14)))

